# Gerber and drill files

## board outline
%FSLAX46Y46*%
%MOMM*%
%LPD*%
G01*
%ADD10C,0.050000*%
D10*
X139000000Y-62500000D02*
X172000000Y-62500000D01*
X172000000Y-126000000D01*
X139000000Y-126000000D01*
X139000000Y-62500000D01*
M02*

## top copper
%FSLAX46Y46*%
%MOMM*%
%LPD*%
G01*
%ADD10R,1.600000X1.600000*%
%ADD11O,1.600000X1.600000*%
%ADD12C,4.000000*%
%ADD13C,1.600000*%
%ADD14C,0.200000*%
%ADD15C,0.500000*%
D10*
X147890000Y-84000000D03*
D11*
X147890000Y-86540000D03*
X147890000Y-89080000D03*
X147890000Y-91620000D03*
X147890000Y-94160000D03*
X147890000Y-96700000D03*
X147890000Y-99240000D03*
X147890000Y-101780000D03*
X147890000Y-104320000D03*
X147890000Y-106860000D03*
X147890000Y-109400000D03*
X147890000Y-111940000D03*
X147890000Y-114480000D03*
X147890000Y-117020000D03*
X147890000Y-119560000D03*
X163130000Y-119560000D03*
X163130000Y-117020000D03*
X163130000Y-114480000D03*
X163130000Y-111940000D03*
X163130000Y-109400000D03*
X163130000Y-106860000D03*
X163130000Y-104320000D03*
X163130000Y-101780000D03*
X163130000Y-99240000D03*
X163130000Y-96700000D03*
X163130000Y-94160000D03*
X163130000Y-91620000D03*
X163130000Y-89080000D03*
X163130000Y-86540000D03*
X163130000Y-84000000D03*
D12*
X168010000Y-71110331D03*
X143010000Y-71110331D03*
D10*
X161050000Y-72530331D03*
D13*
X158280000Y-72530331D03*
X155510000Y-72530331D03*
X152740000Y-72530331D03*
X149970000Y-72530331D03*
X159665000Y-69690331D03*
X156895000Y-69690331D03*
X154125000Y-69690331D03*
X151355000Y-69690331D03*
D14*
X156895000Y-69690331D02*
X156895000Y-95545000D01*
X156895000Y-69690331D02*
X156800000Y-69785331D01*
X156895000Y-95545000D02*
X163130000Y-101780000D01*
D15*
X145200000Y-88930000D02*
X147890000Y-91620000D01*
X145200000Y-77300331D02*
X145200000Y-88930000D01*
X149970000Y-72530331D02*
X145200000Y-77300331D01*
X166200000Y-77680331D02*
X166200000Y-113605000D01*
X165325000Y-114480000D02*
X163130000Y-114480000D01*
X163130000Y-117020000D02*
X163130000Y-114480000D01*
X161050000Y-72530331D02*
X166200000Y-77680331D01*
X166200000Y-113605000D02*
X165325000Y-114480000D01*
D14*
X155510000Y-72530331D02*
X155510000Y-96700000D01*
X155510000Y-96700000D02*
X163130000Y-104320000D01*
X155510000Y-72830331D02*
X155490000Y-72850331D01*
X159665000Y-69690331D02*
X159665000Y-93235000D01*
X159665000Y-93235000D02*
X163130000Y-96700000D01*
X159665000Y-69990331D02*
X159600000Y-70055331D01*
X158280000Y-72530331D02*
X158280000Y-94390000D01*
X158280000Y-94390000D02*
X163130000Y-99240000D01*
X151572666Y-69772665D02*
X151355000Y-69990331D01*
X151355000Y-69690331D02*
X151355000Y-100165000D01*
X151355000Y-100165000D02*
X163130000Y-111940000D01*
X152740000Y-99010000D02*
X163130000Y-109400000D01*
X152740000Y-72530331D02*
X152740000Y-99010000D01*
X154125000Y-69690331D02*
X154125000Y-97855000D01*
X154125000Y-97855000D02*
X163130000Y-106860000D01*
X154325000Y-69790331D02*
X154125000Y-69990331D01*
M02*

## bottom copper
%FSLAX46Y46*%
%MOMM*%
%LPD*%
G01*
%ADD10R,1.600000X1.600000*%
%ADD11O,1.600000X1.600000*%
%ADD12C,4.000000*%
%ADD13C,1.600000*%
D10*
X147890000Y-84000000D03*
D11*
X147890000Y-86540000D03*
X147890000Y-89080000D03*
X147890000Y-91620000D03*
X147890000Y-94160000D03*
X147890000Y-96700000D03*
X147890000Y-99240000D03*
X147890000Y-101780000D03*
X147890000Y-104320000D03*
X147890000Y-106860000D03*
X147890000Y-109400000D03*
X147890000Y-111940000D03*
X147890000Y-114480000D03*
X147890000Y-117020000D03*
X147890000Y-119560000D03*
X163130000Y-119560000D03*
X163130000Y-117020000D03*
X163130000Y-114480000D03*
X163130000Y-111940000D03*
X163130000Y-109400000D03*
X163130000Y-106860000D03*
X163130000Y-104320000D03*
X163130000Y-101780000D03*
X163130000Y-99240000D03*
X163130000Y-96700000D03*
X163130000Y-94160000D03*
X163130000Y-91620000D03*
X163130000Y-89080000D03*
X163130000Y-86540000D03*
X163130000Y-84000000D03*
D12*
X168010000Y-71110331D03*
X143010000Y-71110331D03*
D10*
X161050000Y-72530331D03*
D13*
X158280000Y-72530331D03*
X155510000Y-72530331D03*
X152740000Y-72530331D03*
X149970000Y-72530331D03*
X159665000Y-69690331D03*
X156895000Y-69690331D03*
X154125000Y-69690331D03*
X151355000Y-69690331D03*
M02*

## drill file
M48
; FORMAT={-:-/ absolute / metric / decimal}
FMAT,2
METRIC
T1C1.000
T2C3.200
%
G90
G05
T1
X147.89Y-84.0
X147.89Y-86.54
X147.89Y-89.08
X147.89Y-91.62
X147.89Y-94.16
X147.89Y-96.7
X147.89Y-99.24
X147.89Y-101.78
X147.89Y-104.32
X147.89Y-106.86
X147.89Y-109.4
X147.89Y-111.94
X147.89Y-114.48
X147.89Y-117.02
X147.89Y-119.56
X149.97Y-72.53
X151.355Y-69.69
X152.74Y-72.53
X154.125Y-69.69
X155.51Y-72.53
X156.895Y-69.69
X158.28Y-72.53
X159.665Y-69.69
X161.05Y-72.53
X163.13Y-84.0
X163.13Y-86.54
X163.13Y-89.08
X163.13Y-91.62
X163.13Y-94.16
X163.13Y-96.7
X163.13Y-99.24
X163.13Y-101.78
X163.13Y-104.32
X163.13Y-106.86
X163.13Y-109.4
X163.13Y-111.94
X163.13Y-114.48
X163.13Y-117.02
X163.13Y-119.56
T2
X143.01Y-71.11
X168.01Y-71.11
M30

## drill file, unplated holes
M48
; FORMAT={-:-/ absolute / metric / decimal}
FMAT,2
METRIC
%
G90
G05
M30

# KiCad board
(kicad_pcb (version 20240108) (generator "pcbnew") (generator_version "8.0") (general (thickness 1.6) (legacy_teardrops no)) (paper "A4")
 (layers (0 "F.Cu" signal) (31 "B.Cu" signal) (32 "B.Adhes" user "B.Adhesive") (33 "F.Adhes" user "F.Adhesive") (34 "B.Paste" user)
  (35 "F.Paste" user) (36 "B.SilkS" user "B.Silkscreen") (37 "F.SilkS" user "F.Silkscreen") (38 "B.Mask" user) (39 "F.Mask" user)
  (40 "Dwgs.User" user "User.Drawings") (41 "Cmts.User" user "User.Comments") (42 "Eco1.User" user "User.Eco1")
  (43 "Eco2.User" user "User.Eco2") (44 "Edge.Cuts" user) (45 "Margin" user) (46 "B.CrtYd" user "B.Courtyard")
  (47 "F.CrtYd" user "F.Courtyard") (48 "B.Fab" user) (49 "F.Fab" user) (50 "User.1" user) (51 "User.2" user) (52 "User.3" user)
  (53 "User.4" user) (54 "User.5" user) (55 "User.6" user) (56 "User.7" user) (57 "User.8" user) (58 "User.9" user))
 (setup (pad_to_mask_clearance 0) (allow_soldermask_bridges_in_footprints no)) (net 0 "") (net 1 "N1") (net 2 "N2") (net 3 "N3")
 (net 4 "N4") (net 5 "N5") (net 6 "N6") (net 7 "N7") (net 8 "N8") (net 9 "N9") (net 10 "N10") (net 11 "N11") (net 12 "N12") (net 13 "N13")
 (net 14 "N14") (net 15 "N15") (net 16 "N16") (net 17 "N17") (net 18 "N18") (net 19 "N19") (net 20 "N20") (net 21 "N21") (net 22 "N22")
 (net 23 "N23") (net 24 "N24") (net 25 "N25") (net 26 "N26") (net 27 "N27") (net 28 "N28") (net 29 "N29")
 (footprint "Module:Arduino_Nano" (layer "F.Cu") (at 147.89 84)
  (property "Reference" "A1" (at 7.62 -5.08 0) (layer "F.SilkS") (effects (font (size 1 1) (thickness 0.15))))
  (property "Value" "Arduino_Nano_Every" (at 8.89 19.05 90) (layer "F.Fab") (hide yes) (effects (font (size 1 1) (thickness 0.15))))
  (pad "1" thru_hole rect (at 0 0) (size 1.6 1.6) (drill 1) (layers "*.Cu" "*.Mask") (remove_unused_layers no) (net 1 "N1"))
  (pad "2" thru_hole oval (at 0 2.54) (size 1.6 1.6) (drill 1) (layers "*.Cu" "*.Mask") (remove_unused_layers no) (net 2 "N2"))
  (pad "3" thru_hole oval (at 0 5.08) (size 1.6 1.6) (drill 1) (layers "*.Cu" "*.Mask") (remove_unused_layers no) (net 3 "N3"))
  (pad "4" thru_hole oval (at 0 7.62) (size 1.6 1.6) (drill 1) (layers "*.Cu" "*.Mask") (remove_unused_layers no) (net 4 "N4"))
  (pad "5" thru_hole oval (at 0 10.16) (size 1.6 1.6) (drill 1) (layers "*.Cu" "*.Mask") (remove_unused_layers no) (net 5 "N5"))
  (pad "6" thru_hole oval (at 0 12.7) (size 1.6 1.6) (drill 1) (layers "*.Cu" "*.Mask") (remove_unused_layers no) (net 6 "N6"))
  (pad "7" thru_hole oval (at 0 15.24) (size 1.6 1.6) (drill 1) (layers "*.Cu" "*.Mask") (remove_unused_layers no) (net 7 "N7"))
  (pad "8" thru_hole oval (at 0 17.78) (size 1.6 1.6) (drill 1) (layers "*.Cu" "*.Mask") (remove_unused_layers no) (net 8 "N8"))
  (pad "9" thru_hole oval (at 0 20.32) (size 1.6 1.6) (drill 1) (layers "*.Cu" "*.Mask") (remove_unused_layers no) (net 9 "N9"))
  (pad "10" thru_hole oval (at 0 22.86) (size 1.6 1.6) (drill 1) (layers "*.Cu" "*.Mask") (remove_unused_layers no) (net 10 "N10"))
  (pad "11" thru_hole oval (at 0 25.4) (size 1.6 1.6) (drill 1) (layers "*.Cu" "*.Mask") (remove_unused_layers no) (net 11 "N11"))
  (pad "12" thru_hole oval (at 0 27.94) (size 1.6 1.6) (drill 1) (layers "*.Cu" "*.Mask") (remove_unused_layers no) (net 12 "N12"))
  (pad "13" thru_hole oval (at 0 30.48) (size 1.6 1.6) (drill 1) (layers "*.Cu" "*.Mask") (remove_unused_layers no) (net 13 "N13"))
  (pad "14" thru_hole oval (at 0 33.02) (size 1.6 1.6) (drill 1) (layers "*.Cu" "*.Mask") (remove_unused_layers no) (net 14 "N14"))
  (pad "15" thru_hole oval (at 0 35.56) (size 1.6 1.6) (drill 1) (layers "*.Cu" "*.Mask") (remove_unused_layers no) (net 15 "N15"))
  (pad "16" thru_hole oval (at 15.24 35.56) (size 1.6 1.6) (drill 1) (layers "*.Cu" "*.Mask") (remove_unused_layers no) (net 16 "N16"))
  (pad "17" thru_hole oval (at 15.24 33.02) (size 1.6 1.6) (drill 1) (layers "*.Cu" "*.Mask") (remove_unused_layers no) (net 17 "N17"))
  (pad "18" thru_hole oval (at 15.24 30.48) (size 1.6 1.6) (drill 1) (layers "*.Cu" "*.Mask") (remove_unused_layers no) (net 17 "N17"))
  (pad "19" thru_hole oval (at 15.24 27.94) (size 1.6 1.6) (drill 1) (layers "*.Cu" "*.Mask") (remove_unused_layers no) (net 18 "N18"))
  (pad "20" thru_hole oval (at 15.24 25.4) (size 1.6 1.6) (drill 1) (layers "*.Cu" "*.Mask") (remove_unused_layers no) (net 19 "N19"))
  (pad "21" thru_hole oval (at 15.24 22.86) (size 1.6 1.6) (drill 1) (layers "*.Cu" "*.Mask") (remove_unused_layers no) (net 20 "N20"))
  (pad "22" thru_hole oval (at 15.24 20.32) (size 1.6 1.6) (drill 1) (layers "*.Cu" "*.Mask") (remove_unused_layers no) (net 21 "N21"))
  (pad "23" thru_hole oval (at 15.24 17.78) (size 1.6 1.6) (drill 1) (layers "*.Cu" "*.Mask") (remove_unused_layers no) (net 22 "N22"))
  (pad "24" thru_hole oval (at 15.24 15.24) (size 1.6 1.6) (drill 1) (layers "*.Cu" "*.Mask") (remove_unused_layers no) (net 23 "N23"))
  (pad "25" thru_hole oval (at 15.24 12.7) (size 1.6 1.6) (drill 1) (layers "*.Cu" "*.Mask") (remove_unused_layers no) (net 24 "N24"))
  (pad "26" thru_hole oval (at 15.24 10.16) (size 1.6 1.6) (drill 1) (layers "*.Cu" "*.Mask") (remove_unused_layers no) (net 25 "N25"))
  (pad "27" thru_hole oval (at 15.24 7.62) (size 1.6 1.6) (drill 1) (layers "*.Cu" "*.Mask") (remove_unused_layers no) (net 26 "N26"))
  (pad "28" thru_hole oval (at 15.24 5.08) (size 1.6 1.6) (drill 1) (layers "*.Cu" "*.Mask") (remove_unused_layers no) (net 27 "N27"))
  (pad "29" thru_hole oval (at 15.24 2.54) (size 1.6 1.6) (drill 1) (layers "*.Cu" "*.Mask") (remove_unused_layers no) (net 4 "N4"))
  (pad "30" thru_hole oval (at 15.24 0) (size 1.6 1.6) (drill 1) (layers "*.Cu" "*.Mask") (remove_unused_layers no) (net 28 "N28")))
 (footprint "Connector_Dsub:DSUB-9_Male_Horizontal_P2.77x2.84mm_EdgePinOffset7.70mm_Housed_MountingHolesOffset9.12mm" (layer "F.Cu")
  (at 161.05 72.530331 180)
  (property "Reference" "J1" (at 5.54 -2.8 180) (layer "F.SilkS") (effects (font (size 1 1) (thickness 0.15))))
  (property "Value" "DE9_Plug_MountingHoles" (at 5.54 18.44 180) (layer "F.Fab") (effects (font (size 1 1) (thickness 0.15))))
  (pad "0" thru_hole circle (at -6.96 1.42 180) (size 4 4) (drill 3.2) (layers "*.Cu" "*.Mask") (remove_unused_layers no) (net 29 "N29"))
  (pad "0" thru_hole circle (at 18.04 1.42 180) (size 4 4) (drill 3.2) (layers "*.Cu" "*.Mask") (remove_unused_layers no) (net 29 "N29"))
  (pad "1" thru_hole rect (at 0 0 180) (size 1.6 1.6) (drill 1) (layers "*.Cu" "*.Mask") (remove_unused_layers no) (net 17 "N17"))
  (pad "2" thru_hole circle (at 2.77 0 180) (size 1.6 1.6) (drill 1) (layers "*.Cu" "*.Mask") (remove_unused_layers no) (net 23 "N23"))
  (pad "3" thru_hole circle (at 5.54 0 180) (size 1.6 1.6) (drill 1) (layers "*.Cu" "*.Mask") (remove_unused_layers no) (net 21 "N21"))
  (pad "4" thru_hole circle (at 8.31 0 180) (size 1.6 1.6) (drill 1) (layers "*.Cu" "*.Mask") (remove_unused_layers no) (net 19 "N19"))
  (pad "5" thru_hole circle (at 11.08 0 180) (size 1.6 1.6) (drill 1) (layers "*.Cu" "*.Mask") (remove_unused_layers no) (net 4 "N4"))
  (pad "6" thru_hole circle (at 1.385 2.84 180) (size 1.6 1.6) (drill 1) (layers "*.Cu" "*.Mask") (remove_unused_layers no) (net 24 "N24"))
  (pad "7" thru_hole circle (at 4.155 2.84 180) (size 1.6 1.6) (drill 1) (layers "*.Cu" "*.Mask") (remove_unused_layers no) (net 22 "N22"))
  (pad "8" thru_hole circle (at 6.925 2.84 180) (size 1.6 1.6) (drill 1) (layers "*.Cu" "*.Mask") (remove_unused_layers no) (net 20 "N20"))
  (pad "9" thru_hole circle (at 9.695 2.84 180) (size 1.6 1.6) (drill 1) (layers "*.Cu" "*.Mask") (remove_unused_layers no) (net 18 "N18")))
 (gr_rect (start 139 62.5) (end 172 126) (stroke (width 0.05) (type default)) (fill none) (layer "Edge.Cuts"))
 (segment (start 156.895 69.690331) (end 156.895 95.545) (width 0.2) (layer "F.Cu") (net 22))
 (segment (start 156.895 69.690331) (end 156.8 69.785331) (width 0.2) (layer "F.Cu") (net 22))
 (segment (start 156.895 95.545) (end 163.13 101.78) (width 0.2) (layer "F.Cu") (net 22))
 (segment (start 145.2 88.93) (end 147.89 91.62) (width 0.5) (layer "F.Cu") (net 4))
 (segment (start 145.2 77.300331) (end 145.2 88.93) (width 0.5) (layer "F.Cu") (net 4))
 (segment (start 149.97 72.530331) (end 145.2 77.300331) (width 0.5) (layer "F.Cu") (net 4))
 (segment (start 166.2 77.680331) (end 166.2 113.605) (width 0.5) (layer "F.Cu") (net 17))
 (segment (start 165.325 114.48) (end 163.13 114.48) (width 0.5) (layer "F.Cu") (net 17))
 (segment (start 163.13 117.02) (end 163.13 114.48) (width 0.5) (layer "F.Cu") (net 17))
 (segment (start 161.05 72.530331) (end 166.2 77.680331) (width 0.5) (layer "F.Cu") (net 17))
 (segment (start 166.2 113.605) (end 165.325 114.48) (width 0.5) (layer "F.Cu") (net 17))
 (segment (start 155.51 72.530331) (end 155.51 96.7) (width 0.2) (layer "F.Cu") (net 21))
 (segment (start 155.51 96.7) (end 163.13 104.32) (width 0.2) (layer "F.Cu") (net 21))
 (segment (start 155.51 72.830331) (end 155.49 72.850331) (width 0.2) (layer "F.Cu") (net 21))
 (segment (start 159.665 69.690331) (end 159.665 93.235) (width 0.2) (layer "F.Cu") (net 24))
 (segment (start 159.665 93.235) (end 163.13 96.7) (width 0.2) (layer "F.Cu") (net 24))
 (segment (start 159.665 69.990331) (end 159.6 70.055331) (width 0.2) (layer "F.Cu") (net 24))
 (segment (start 158.28 72.530331) (end 158.28 94.39) (width 0.2) (layer "F.Cu") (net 23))
 (segment (start 158.28 94.39) (end 163.13 99.24) (width 0.2) (layer "F.Cu") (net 23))
 (segment (start 151.572666 69.772665) (end 151.355 69.990331) (width 0.2) (layer "F.Cu") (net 18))
 (segment (start 151.355 69.690331) (end 151.355 100.165) (width 0.2) (layer "F.Cu") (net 18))
 (segment (start 151.355 100.165) (end 163.13 111.94) (width 0.2) (layer "F.Cu") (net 18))
 (segment (start 152.74 99.01) (end 163.13 109.4) (width 0.2) (layer "F.Cu") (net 19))
 (segment (start 152.74 72.530331) (end 152.74 99.01) (width 0.2) (layer "F.Cu") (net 19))
 (segment (start 154.125 69.690331) (end 154.125 97.855) (width 0.2) (layer "F.Cu") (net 20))
 (segment (start 154.125 97.855) (end 163.13 106.86) (width 0.2) (layer "F.Cu") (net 20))
 (segment (start 154.325 69.790331) (end 154.125 69.990331) (width 0.2) (layer "F.Cu") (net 20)))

